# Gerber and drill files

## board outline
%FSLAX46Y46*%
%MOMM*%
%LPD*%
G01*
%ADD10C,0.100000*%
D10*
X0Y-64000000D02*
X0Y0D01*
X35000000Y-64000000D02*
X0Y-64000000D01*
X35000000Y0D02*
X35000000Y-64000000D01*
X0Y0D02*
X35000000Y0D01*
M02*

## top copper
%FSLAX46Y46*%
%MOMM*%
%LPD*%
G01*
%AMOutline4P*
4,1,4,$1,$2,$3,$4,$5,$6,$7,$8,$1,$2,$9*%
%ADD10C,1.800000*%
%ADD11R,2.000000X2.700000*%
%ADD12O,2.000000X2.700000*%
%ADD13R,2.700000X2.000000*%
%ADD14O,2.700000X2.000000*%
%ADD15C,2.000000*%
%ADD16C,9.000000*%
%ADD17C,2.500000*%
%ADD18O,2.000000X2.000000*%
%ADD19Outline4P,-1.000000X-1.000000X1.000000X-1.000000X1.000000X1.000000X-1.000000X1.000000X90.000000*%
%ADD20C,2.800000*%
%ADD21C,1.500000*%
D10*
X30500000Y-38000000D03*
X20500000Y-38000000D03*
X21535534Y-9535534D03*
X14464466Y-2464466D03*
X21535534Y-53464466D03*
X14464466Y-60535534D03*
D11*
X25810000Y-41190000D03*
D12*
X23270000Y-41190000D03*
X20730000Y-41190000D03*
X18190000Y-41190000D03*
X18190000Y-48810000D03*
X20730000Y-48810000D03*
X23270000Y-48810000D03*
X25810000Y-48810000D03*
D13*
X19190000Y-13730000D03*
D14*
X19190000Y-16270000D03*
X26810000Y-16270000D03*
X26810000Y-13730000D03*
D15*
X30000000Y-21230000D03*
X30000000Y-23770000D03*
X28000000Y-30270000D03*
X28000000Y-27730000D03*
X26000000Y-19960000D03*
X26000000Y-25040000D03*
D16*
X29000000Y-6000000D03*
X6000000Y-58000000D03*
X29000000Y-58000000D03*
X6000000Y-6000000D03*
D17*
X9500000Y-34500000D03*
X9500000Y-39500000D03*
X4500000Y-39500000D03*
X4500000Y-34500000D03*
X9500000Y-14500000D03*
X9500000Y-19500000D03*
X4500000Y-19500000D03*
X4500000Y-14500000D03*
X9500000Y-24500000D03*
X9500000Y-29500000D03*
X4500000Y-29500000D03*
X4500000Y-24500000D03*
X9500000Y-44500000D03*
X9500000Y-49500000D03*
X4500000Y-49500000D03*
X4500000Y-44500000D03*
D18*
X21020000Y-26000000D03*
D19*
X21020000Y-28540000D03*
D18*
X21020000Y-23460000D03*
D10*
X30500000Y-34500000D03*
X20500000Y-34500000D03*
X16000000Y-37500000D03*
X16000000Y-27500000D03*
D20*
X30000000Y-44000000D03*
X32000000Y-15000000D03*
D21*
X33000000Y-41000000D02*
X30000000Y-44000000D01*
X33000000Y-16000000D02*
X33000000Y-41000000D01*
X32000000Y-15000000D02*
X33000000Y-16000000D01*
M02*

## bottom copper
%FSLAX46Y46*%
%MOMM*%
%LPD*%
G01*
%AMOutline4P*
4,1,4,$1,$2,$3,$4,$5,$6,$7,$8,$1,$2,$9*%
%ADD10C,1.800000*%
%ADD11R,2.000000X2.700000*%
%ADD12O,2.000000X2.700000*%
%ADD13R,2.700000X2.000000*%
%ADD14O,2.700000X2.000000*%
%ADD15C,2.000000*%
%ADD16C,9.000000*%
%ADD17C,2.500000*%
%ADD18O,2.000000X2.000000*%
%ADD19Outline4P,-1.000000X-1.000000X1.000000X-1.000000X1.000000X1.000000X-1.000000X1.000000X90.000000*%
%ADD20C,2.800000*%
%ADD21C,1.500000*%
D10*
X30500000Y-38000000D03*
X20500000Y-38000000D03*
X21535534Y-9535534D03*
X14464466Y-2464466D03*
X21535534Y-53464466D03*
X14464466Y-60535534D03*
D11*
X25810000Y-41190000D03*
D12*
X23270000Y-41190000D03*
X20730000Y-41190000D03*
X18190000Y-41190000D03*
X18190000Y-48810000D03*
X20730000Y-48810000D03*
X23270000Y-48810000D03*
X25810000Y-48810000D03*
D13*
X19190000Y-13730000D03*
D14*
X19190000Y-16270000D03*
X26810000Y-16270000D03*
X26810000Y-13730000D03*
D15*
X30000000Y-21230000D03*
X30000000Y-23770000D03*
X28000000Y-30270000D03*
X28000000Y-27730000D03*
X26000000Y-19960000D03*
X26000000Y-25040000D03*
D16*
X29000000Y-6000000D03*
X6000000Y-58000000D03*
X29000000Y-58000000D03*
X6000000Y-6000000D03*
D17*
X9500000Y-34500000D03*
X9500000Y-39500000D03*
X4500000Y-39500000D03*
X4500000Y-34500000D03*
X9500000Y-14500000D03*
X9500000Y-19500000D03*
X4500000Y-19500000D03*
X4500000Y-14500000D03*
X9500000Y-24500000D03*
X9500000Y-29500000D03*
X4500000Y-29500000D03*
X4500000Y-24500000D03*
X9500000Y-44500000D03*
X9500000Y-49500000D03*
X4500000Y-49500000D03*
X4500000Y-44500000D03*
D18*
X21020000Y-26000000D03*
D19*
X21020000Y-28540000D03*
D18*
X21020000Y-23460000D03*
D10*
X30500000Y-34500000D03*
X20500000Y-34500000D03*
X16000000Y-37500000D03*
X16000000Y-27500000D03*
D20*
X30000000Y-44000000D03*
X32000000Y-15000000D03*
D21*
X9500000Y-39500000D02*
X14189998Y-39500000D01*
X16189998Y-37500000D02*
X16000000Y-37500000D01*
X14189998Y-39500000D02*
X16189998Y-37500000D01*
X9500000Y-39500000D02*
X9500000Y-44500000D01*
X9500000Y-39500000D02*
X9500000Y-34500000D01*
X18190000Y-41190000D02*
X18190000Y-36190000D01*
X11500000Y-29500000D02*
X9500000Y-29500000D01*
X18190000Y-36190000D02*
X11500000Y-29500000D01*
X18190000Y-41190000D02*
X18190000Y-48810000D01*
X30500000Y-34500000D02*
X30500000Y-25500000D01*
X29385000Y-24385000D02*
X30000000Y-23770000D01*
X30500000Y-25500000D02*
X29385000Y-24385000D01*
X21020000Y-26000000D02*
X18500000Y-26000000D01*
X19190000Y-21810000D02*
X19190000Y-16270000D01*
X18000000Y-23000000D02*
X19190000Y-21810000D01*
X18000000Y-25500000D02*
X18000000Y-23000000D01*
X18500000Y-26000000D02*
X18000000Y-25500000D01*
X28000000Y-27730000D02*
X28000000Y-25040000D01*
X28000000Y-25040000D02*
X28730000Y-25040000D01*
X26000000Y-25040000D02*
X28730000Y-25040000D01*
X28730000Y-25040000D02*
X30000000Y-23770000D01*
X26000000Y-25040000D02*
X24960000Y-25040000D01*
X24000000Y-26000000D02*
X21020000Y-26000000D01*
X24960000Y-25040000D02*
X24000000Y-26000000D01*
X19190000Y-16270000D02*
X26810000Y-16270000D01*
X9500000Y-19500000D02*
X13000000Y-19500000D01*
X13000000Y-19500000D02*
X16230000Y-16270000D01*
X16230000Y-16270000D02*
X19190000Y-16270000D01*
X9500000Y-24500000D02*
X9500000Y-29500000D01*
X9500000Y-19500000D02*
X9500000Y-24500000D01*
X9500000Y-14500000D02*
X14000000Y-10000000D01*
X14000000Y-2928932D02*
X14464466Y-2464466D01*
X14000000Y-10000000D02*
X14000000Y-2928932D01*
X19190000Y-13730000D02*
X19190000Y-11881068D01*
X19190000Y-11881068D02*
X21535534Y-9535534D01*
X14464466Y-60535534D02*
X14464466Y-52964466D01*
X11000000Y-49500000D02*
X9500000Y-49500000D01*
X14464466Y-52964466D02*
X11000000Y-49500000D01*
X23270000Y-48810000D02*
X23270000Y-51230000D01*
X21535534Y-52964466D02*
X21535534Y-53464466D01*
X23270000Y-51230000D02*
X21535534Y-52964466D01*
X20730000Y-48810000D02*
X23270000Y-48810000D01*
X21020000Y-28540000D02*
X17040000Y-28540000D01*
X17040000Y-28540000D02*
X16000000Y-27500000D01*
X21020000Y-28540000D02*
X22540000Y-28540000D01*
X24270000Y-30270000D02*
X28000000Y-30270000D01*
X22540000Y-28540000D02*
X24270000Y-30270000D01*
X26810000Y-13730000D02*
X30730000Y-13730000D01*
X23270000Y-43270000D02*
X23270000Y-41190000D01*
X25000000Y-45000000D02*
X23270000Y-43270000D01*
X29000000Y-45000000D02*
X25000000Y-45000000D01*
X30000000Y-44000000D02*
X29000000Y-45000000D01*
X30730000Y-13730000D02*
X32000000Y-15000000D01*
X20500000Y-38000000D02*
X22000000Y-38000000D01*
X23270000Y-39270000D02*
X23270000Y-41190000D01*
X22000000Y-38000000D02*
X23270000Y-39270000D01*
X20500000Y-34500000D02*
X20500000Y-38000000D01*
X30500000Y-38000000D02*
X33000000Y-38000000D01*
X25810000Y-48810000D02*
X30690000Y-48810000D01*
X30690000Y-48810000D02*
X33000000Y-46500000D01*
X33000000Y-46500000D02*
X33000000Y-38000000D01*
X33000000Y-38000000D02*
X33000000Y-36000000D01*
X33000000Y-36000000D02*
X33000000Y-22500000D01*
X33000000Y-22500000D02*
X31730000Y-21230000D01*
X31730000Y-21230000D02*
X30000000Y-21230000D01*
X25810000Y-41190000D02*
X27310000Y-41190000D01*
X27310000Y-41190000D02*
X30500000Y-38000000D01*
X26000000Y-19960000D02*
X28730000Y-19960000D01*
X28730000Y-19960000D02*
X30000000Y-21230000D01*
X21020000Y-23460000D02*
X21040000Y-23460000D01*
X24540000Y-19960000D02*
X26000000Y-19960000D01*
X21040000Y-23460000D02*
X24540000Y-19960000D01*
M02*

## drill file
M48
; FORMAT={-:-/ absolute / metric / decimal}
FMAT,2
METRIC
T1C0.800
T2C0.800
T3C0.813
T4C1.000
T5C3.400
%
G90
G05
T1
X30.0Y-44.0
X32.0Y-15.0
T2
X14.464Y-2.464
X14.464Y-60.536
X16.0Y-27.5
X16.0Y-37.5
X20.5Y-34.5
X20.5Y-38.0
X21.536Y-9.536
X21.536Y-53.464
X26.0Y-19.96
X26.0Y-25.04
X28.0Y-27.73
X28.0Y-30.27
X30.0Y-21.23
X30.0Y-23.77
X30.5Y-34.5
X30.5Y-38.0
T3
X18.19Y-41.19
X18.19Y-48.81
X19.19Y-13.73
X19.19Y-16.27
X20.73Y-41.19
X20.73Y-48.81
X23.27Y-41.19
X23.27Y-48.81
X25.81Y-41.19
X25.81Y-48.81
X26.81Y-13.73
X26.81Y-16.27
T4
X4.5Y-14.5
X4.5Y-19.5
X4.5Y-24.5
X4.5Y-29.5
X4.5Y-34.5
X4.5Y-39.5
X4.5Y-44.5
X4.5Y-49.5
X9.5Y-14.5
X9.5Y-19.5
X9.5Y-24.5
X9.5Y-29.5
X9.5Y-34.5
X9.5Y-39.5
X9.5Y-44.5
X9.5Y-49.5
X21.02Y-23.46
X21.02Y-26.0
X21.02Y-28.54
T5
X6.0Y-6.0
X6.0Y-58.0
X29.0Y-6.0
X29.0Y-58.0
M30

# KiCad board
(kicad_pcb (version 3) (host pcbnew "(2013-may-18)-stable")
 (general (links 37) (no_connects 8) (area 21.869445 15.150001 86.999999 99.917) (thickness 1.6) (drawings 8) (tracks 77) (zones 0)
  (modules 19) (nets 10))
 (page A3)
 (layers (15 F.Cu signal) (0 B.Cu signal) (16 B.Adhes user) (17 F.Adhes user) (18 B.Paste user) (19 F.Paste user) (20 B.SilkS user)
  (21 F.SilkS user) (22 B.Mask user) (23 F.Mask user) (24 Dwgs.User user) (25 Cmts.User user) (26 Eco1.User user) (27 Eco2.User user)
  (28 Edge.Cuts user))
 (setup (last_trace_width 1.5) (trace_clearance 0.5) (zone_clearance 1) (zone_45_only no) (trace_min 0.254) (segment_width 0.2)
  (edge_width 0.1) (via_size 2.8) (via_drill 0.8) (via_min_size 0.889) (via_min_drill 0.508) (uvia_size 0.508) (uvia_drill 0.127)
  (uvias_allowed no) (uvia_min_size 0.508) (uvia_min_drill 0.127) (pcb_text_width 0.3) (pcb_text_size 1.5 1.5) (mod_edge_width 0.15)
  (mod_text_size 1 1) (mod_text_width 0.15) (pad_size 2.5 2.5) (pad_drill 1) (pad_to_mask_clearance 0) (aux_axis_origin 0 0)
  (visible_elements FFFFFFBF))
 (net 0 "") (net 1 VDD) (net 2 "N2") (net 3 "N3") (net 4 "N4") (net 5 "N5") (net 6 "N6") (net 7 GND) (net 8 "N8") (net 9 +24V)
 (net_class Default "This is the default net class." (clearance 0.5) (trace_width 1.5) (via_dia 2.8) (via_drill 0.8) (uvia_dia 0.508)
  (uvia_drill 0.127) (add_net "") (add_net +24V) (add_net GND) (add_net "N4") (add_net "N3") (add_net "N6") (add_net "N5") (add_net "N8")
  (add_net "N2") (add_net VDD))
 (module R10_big (layer F.Cu) (at 25.5 38 180) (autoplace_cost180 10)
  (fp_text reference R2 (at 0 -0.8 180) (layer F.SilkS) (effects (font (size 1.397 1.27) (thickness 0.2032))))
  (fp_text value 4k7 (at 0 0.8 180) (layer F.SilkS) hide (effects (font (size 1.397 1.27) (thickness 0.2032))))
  (pad 1 thru_hole circle (at -5 0 180) (size 1.8 1.8) (drill 0.8) (layers *.Cu *.Mask F.SilkS) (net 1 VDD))
  (pad 2 thru_hole circle (at 5 0 180) (size 1.8 1.8) (drill 0.8) (layers *.Cu *.Mask F.SilkS) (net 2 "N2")))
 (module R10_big (layer F.Cu) (at 18 6 135) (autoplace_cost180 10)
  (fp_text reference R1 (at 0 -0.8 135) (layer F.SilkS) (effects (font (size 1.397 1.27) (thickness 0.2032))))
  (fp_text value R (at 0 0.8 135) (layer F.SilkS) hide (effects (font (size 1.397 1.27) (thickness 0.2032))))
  (pad 1 thru_hole circle (at -5 0 135) (size 1.8 1.8) (drill 0.8) (layers *.Cu *.Mask F.SilkS) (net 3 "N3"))
  (pad 2 thru_hole circle (at 5 0 135) (size 1.8 1.8) (drill 0.8) (layers *.Cu *.Mask F.SilkS) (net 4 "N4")))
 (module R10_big (layer F.Cu) (at 18 57 225) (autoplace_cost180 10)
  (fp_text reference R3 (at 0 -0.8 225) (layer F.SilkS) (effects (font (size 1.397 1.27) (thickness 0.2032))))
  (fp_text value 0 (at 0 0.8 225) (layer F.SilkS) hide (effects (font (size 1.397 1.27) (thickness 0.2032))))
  (pad 1 thru_hole circle (at -5 0 225) (size 1.8 1.8) (drill 0.8) (layers *.Cu *.Mask F.SilkS) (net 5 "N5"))
  (pad 2 thru_hole circle (at 5 0 225) (size 1.8 1.8) (drill 0.8) (layers *.Cu *.Mask F.SilkS) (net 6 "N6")))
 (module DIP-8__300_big (layer F.Cu) (at 22 45 180)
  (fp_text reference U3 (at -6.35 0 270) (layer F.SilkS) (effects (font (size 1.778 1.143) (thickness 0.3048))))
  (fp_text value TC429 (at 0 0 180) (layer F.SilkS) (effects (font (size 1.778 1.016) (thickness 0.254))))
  (pad 1 thru_hole rect (at -3.81 3.81 180) (size 2 2.7) (drill 0.8128) (layers *.Cu *.Mask F.SilkS) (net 1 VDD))
  (pad 2 thru_hole oval (at -1.27 3.81 180) (size 2 2.7) (drill 0.8128) (layers *.Cu *.Mask F.SilkS) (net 2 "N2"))
  (pad 3 thru_hole oval (at 1.27 3.81 180) (size 2 2.7) (drill 0.8128) (layers *.Cu *.Mask F.SilkS))
  (pad 4 thru_hole oval (at 3.81 3.81 180) (size 2 2.7) (drill 0.8128) (layers *.Cu *.Mask F.SilkS) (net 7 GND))
  (pad 5 thru_hole oval (at 3.81 -3.81 180) (size 2 2.7) (drill 0.8128) (layers *.Cu *.Mask F.SilkS) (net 7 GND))
  (pad 6 thru_hole oval (at 1.27 -3.81 180) (size 2 2.7) (drill 0.8128) (layers *.Cu *.Mask F.SilkS) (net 5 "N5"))
  (pad 7 thru_hole oval (at -1.27 -3.81 180) (size 2 2.7) (drill 0.8128) (layers *.Cu *.Mask F.SilkS) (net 5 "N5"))
  (pad 8 thru_hole oval (at -3.81 -3.81 180) (size 2 2.7) (drill 0.8128) (layers *.Cu *.Mask F.SilkS) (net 1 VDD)))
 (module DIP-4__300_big (layer F.Cu) (at 23 15 270)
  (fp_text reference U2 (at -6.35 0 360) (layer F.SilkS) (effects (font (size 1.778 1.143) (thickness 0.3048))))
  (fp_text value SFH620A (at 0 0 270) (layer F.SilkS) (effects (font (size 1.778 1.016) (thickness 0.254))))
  (pad 1 thru_hole rect (at -1.27 3.81 270) (size 2 2.7) (drill 0.8128) (layers *.Cu *.Mask F.SilkS) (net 3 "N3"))
  (pad 2 thru_hole oval (at 1.27 3.81 270) (size 2 2.7) (drill 0.8128) (layers *.Cu *.Mask F.SilkS) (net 7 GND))
  (pad 3 thru_hole oval (at 1.27 -3.81 270) (size 2 2.7) (drill 0.8128) (layers *.Cu *.Mask F.SilkS) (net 7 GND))
  (pad 4 thru_hole oval (at -1.27 -3.81 270) (size 2 2.7) (drill 0.8128) (layers *.Cu *.Mask F.SilkS) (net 2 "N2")))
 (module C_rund (layer F.Cu) (at 30 22.5 270)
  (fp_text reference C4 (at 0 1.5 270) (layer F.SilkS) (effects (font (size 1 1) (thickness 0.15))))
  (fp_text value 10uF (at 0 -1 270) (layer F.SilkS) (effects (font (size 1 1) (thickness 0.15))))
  (pad 1 thru_hole circle (at -1.27 0 270) (size 2 2) (drill 0.8) (layers *.Cu *.Mask F.SilkS) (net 1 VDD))
  (pad 2 thru_hole circle (at 1.27 0 270) (size 2 2) (drill 0.8) (layers *.Cu *.Mask F.SilkS) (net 7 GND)))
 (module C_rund (layer F.Cu) (at 28 29 90)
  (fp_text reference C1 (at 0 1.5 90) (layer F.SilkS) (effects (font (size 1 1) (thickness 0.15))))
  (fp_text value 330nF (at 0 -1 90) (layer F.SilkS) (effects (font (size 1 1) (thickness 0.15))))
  (pad 1 thru_hole circle (at -1.27 0 90) (size 2 2) (drill 0.8) (layers *.Cu *.Mask F.SilkS) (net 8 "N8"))
  (pad 2 thru_hole circle (at 1.27 0 90) (size 2 2) (drill 0.8) (layers *.Cu *.Mask F.SilkS) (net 7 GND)))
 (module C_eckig (layer F.Cu) (at 26 22.5 270)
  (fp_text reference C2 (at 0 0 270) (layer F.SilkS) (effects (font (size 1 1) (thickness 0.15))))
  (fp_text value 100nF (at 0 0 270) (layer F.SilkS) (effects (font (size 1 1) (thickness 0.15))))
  (pad 1 thru_hole circle (at -2.54 0 270) (size 2 2) (drill 0.8) (layers *.Cu *.Mask F.SilkS) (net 1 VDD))
  (pad 2 thru_hole circle (at 2.54 0 270) (size 2 2) (drill 0.8) (layers *.Cu *.Mask F.SilkS) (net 7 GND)))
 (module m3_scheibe (layer F.Cu) (at 29 6)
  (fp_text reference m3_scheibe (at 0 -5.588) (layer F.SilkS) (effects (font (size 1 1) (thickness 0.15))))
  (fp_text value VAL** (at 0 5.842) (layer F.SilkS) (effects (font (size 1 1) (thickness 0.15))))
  (pad 1 thru_hole circle (at 0 0) (size 9 9) (drill 3.4) (layers *.Cu *.Mask F.SilkS) (clearance 1)))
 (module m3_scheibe (layer F.Cu) (at 6 58)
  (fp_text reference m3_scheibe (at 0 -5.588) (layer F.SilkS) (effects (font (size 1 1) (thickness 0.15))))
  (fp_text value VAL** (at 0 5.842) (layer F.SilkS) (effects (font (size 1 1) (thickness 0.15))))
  (pad 1 thru_hole circle (at 0 0) (size 9 9) (drill 3.4) (layers *.Cu *.Mask F.SilkS) (clearance 1)))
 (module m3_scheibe (layer F.Cu) (at 29 58)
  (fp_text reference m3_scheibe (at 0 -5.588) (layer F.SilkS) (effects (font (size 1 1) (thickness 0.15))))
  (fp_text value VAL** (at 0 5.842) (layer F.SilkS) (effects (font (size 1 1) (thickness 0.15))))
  (pad 1 thru_hole circle (at 0 0) (size 9 9) (drill 3.4) (layers *.Cu *.Mask F.SilkS) (clearance 1)))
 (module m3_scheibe (layer F.Cu) (at 6 6)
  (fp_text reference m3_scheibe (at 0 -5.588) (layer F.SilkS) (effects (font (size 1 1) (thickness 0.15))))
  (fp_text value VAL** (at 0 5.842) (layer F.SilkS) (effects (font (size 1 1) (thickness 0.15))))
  (pad 1 thru_hole circle (at 0 0) (size 9 9) (drill 3.4) (layers *.Cu *.Mask F.SilkS) (clearance 1)))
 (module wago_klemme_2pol (layer F.Cu) (at 7 37 270)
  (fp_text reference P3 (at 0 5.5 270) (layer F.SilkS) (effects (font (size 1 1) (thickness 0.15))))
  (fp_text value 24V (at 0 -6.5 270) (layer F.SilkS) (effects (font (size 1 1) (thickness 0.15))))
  (pad 1 thru_hole circle (at -2.5 -2.5 270) (size 2.5 2.5) (drill 1) (layers *.Cu *.Mask F.SilkS) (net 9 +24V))
  (pad 2 thru_hole circle (at 2.5 -2.5 270) (size 2.5 2.5) (drill 1) (layers *.Cu *.Mask F.SilkS) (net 9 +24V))
  (pad 2 thru_hole circle (at 2.5 2.5 270) (size 2.5 2.5) (drill 1) (layers *.Cu *.Mask F.SilkS) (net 9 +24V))
  (pad 1 thru_hole circle (at -2.5 2.5 270) (size 2.5 2.5) (drill 1) (layers *.Cu *.Mask F.SilkS) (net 9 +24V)))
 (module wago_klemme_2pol (layer F.Cu) (at 7 17 270)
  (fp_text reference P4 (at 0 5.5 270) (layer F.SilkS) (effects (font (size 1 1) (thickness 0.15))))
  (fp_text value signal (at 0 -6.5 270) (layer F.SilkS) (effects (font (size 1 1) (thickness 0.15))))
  (pad 1 thru_hole circle (at -2.5 -2.5 270) (size 2.5 2.5) (drill 1) (layers *.Cu *.Mask F.SilkS) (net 4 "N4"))
  (pad 2 thru_hole circle (at 2.5 -2.5 270) (size 2.5 2.5) (drill 1) (layers *.Cu *.Mask F.SilkS) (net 7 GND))
  (pad 2 thru_hole circle (at 2.5 2.5 270) (size 2.5 2.5) (drill 1) (layers *.Cu *.Mask F.SilkS) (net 7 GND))
  (pad 1 thru_hole circle (at -2.5 2.5 270) (size 2.5 2.5) (drill 1) (layers *.Cu *.Mask F.SilkS) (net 4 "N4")))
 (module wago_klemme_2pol (layer F.Cu) (at 7 27 270)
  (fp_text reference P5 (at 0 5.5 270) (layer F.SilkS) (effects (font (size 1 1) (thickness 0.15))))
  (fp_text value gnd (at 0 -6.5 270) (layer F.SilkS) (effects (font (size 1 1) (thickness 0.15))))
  (pad 1 thru_hole circle (at -2.5 -2.5 270) (size 2.5 2.5) (drill 1) (layers *.Cu *.Mask F.SilkS) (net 7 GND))
  (pad 2 thru_hole circle (at 2.5 -2.5 270) (size 2.5 2.5) (drill 1) (layers *.Cu *.Mask F.SilkS) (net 7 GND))
  (pad 2 thru_hole circle (at 2.5 2.5 270) (size 2.5 2.5) (drill 1) (layers *.Cu *.Mask F.SilkS) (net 7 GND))
  (pad 1 thru_hole circle (at -2.5 2.5 270) (size 2.5 2.5) (drill 1) (layers *.Cu *.Mask F.SilkS) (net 7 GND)))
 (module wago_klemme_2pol (layer F.Cu) (at 7 47 270)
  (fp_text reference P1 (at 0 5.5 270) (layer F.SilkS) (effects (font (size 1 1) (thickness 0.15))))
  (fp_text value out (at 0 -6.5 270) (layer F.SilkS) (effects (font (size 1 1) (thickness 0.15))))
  (pad 1 thru_hole circle (at -2.5 -2.5 270) (size 2.5 2.5) (drill 1) (layers *.Cu *.Mask F.SilkS) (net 9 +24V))
  (pad 2 thru_hole circle (at 2.5 -2.5 270) (size 2.5 2.5) (drill 1) (layers *.Cu *.Mask F.SilkS) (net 6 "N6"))
  (pad 2 thru_hole circle (at 2.5 2.5 270) (size 2.5 2.5) (drill 1) (layers *.Cu *.Mask F.SilkS) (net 6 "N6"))
  (pad 1 thru_hole circle (at -2.5 2.5 270) (size 2.5 2.5) (drill 1) (layers *.Cu *.Mask F.SilkS) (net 9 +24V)))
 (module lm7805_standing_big (layer F.Cu) (at 21 26 90)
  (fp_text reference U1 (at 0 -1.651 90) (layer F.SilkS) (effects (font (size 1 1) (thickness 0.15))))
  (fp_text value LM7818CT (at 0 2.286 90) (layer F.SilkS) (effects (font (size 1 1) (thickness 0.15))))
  (pad 2 thru_hole oval (at 0 0.02 90) (size 2 2) (drill 1) (layers *.Cu *.Mask F.SilkS) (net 7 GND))
  (pad 1 thru_hole trapezoid (at -2.54 0.02 90) (size 2 2) (drill 1) (layers *.Cu *.Mask F.SilkS) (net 8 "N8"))
  (pad 3 thru_hole oval (at 2.54 0.02 90) (size 2 2) (drill 1) (layers *.Cu *.Mask F.SilkS) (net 1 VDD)))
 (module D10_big (layer F.Cu) (at 25.5 34.5 180) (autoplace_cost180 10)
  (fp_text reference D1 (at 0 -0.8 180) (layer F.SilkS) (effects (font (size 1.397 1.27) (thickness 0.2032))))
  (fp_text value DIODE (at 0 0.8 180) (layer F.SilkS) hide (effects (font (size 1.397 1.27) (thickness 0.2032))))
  (pad 1 thru_hole circle (at -5 0 180) (size 1.8 1.8) (drill 0.8) (layers *.Cu *.Mask F.SilkS) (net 7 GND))
  (pad 2 thru_hole circle (at 5 0 180) (size 1.8 1.8) (drill 0.8) (layers *.Cu *.Mask F.SilkS) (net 2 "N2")))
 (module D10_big (layer F.Cu) (at 16 32.5 90) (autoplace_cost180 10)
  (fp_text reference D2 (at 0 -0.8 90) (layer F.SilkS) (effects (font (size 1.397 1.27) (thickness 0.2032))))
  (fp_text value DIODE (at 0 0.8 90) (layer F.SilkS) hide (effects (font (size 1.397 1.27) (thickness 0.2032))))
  (pad 1 thru_hole circle (at -5 0 90) (size 1.8 1.8) (drill 0.8) (layers *.Cu *.Mask F.SilkS) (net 9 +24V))
  (pad 2 thru_hole circle (at 5 0 90) (size 1.8 1.8) (drill 0.8) (layers *.Cu *.Mask F.SilkS) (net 8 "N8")))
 (gr_line (start 0 64) (end 0 0) (angle 90) (layer Edge.Cuts) (width 0.1))
 (gr_line (start 35 64) (end 0 64) (angle 90) (layer Edge.Cuts) (width 0.1))
 (gr_line (start 35 0) (end 35 64) (angle 90) (layer Edge.Cuts) (width 0.1))
 (gr_line (start 0 0) (end 35 0) (angle 90) (layer Edge.Cuts) (width 0.1))
 (segment (start 9.5 39.5) (end 14.189998 39.5) (width 1.5) (layer B.Cu) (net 9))
 (segment (start 16.189998 37.5) (end 16 37.5) (width 1.5) (layer B.Cu) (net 9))
 (segment (start 14.189998 39.5) (end 16.189998 37.5) (width 1.5) (layer B.Cu) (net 9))
 (segment (start 9.5 39.5) (end 9.5 44.5) (width 1.5) (layer B.Cu) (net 9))
 (segment (start 9.5 39.5) (end 9.5 34.5) (width 1.5) (layer B.Cu) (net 9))
 (segment (start 18.19 41.19) (end 18.19 36.19) (width 1.5) (layer B.Cu) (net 7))
 (segment (start 11.5 29.5) (end 9.5 29.5) (width 1.5) (layer B.Cu) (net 7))
 (segment (start 18.19 36.19) (end 11.5 29.5) (width 1.5) (layer B.Cu) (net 7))
 (segment (start 18.19 41.19) (end 18.19 48.81) (width 1.5) (layer B.Cu) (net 7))
 (segment (start 30.5 34.5) (end 30.5 25.5) (width 1.5) (layer B.Cu) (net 7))
 (segment (start 29.385 24.385) (end 30 23.77) (width 1.5) (layer B.Cu) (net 7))
 (segment (start 30.5 25.5) (end 29.385 24.385) (width 1.5) (layer B.Cu) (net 7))
 (segment (start 21.02 26) (end 18.5 26) (width 1.5) (layer B.Cu) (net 7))
 (segment (start 19.19 21.81) (end 19.19 16.27) (width 1.5) (layer B.Cu) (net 7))
 (segment (start 18 23) (end 19.19 21.81) (width 1.5) (layer B.Cu) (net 7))
 (segment (start 18 25.5) (end 18 23) (width 1.5) (layer B.Cu) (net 7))
 (segment (start 18.5 26) (end 18 25.5) (width 1.5) (layer B.Cu) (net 7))
 (segment (start 28 27.73) (end 28 25.04) (width 1.5) (layer B.Cu) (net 7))
 (segment (start 28 25.04) (end 28.73 25.04) (width 1.5) (layer B.Cu) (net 7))
 (segment (start 26 25.04) (end 28.73 25.04) (width 1.5) (layer B.Cu) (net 7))
 (segment (start 28.73 25.04) (end 30 23.77) (width 1.5) (layer B.Cu) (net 7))
 (segment (start 26 25.04) (end 24.96 25.04) (width 1.5) (layer B.Cu) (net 7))
 (segment (start 24 26) (end 21.02 26) (width 1.5) (layer B.Cu) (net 7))
 (segment (start 24.96 25.04) (end 24 26) (width 1.5) (layer B.Cu) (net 7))
 (segment (start 19.19 16.27) (end 26.81 16.27) (width 1.5) (layer B.Cu) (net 7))
 (segment (start 9.5 19.5) (end 13 19.5) (width 1.5) (layer B.Cu) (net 7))
 (segment (start 13 19.5) (end 16.23 16.27) (width 1.5) (layer B.Cu) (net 7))
 (segment (start 16.23 16.27) (end 19.19 16.27) (width 1.5) (layer B.Cu) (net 7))
 (segment (start 9.5 24.5) (end 9.5 29.5) (width 1.5) (layer B.Cu) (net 7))
 (segment (start 9.5 19.5) (end 9.5 24.5) (width 1.5) (layer B.Cu) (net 7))
 (segment (start 9.5 14.5) (end 14 10) (width 1.5) (layer B.Cu) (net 4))
 (segment (start 14 2.928932) (end 14.464466 2.464466) (width 1.5) (layer B.Cu) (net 4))
 (segment (start 14 10) (end 14 2.928932) (width 1.5) (layer B.Cu) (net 4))
 (segment (start 19.19 13.73) (end 19.19 11.881068) (width 1.5) (layer B.Cu) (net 3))
 (segment (start 19.19 11.881068) (end 21.535534 9.535534) (width 1.5) (layer B.Cu) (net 3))
 (segment (start 14.464466 60.535534) (end 14.464466 52.964466) (width 1.5) (layer B.Cu) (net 6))
 (segment (start 11 49.5) (end 9.5 49.5) (width 1.5) (layer B.Cu) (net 6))
 (segment (start 14.464466 52.964466) (end 11 49.5) (width 1.5) (layer B.Cu) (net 6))
 (segment (start 23.27 48.81) (end 23.27 51.23) (width 1.5) (layer B.Cu) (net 5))
 (segment (start 21.535534 52.964466) (end 21.535534 53.464466) (width 1.5) (layer B.Cu) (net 5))
 (segment (start 23.27 51.23) (end 21.535534 52.964466) (width 1.5) (layer B.Cu) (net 5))
 (segment (start 20.73 48.81) (end 23.27 48.81) (width 1.5) (layer B.Cu) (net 5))
 (segment (start 21.02 28.54) (end 17.04 28.54) (width 1.5) (layer B.Cu) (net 8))
 (segment (start 17.04 28.54) (end 16 27.5) (width 1.5) (layer B.Cu) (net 8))
 (segment (start 21.02 28.54) (end 22.54 28.54) (width 1.5) (layer B.Cu) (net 8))
 (segment (start 24.27 30.27) (end 28 30.27) (width 1.5) (layer B.Cu) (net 8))
 (segment (start 22.54 28.54) (end 24.27 30.27) (width 1.5) (layer B.Cu) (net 8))
 (segment (start 26.81 13.73) (end 30.73 13.73) (width 1.5) (layer B.Cu) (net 2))
 (segment (start 23.27 43.27) (end 23.27 41.19) (width 1.5) (layer B.Cu) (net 2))
 (segment (start 25 45) (end 23.27 43.27) (width 1.5) (layer B.Cu) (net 2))
 (segment (start 29 45) (end 25 45) (width 1.5) (layer B.Cu) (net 2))
 (segment (start 30 44) (end 29 45) (width 1.5) (layer B.Cu) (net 2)) (via (at 30 44) (size 2.8) (layers F.Cu B.Cu) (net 2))
 (segment (start 33 41) (end 30 44) (width 1.5) (layer F.Cu) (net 2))
 (segment (start 33 16) (end 33 41) (width 1.5) (layer F.Cu) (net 2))
 (segment (start 32 15) (end 33 16) (width 1.5) (layer F.Cu) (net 2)) (via (at 32 15) (size 2.8) (layers F.Cu B.Cu) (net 2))
 (segment (start 30.73 13.73) (end 32 15) (width 1.5) (layer B.Cu) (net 2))
 (segment (start 20.5 38) (end 22 38) (width 1.5) (layer B.Cu) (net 2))
 (segment (start 23.27 39.27) (end 23.27 41.19) (width 1.5) (layer B.Cu) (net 2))
 (segment (start 22 38) (end 23.27 39.27) (width 1.5) (layer B.Cu) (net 2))
 (segment (start 20.5 34.5) (end 20.5 38) (width 1.5) (layer B.Cu) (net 2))
 (segment (start 30.5 38) (end 33 38) (width 1.5) (layer B.Cu) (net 1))
 (segment (start 25.81 48.81) (end 30.69 48.81) (width 1.5) (layer B.Cu) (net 1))
 (segment (start 30.69 48.81) (end 33 46.5) (width 1.5) (layer B.Cu) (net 1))
 (segment (start 33 46.5) (end 33 38) (width 1.5) (layer B.Cu) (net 1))
 (segment (start 33 38) (end 33 36) (width 1.5) (layer B.Cu) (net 1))
 (segment (start 33 36) (end 33 22.5) (width 1.5) (layer B.Cu) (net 1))
 (segment (start 33 22.5) (end 31.73 21.23) (width 1.5) (layer B.Cu) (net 1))
 (segment (start 31.73 21.23) (end 30 21.23) (width 1.5) (layer B.Cu) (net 1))
 (segment (start 25.81 41.19) (end 27.31 41.19) (width 1.5) (layer B.Cu) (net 1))
 (segment (start 27.31 41.19) (end 30.5 38) (width 1.5) (layer B.Cu) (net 1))
 (segment (start 26 19.96) (end 28.73 19.96) (width 1.5) (layer B.Cu) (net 1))
 (segment (start 28.73 19.96) (end 30 21.23) (width 1.5) (layer B.Cu) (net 1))
 (segment (start 21.02 23.46) (end 21.04 23.46) (width 1.5) (layer B.Cu) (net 1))
 (segment (start 24.54 19.96) (end 26 19.96) (width 1.5) (layer B.Cu) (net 1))
 (segment (start 21.04 23.46) (end 24.54 19.96) (width 1.5) (layer B.Cu) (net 1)))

